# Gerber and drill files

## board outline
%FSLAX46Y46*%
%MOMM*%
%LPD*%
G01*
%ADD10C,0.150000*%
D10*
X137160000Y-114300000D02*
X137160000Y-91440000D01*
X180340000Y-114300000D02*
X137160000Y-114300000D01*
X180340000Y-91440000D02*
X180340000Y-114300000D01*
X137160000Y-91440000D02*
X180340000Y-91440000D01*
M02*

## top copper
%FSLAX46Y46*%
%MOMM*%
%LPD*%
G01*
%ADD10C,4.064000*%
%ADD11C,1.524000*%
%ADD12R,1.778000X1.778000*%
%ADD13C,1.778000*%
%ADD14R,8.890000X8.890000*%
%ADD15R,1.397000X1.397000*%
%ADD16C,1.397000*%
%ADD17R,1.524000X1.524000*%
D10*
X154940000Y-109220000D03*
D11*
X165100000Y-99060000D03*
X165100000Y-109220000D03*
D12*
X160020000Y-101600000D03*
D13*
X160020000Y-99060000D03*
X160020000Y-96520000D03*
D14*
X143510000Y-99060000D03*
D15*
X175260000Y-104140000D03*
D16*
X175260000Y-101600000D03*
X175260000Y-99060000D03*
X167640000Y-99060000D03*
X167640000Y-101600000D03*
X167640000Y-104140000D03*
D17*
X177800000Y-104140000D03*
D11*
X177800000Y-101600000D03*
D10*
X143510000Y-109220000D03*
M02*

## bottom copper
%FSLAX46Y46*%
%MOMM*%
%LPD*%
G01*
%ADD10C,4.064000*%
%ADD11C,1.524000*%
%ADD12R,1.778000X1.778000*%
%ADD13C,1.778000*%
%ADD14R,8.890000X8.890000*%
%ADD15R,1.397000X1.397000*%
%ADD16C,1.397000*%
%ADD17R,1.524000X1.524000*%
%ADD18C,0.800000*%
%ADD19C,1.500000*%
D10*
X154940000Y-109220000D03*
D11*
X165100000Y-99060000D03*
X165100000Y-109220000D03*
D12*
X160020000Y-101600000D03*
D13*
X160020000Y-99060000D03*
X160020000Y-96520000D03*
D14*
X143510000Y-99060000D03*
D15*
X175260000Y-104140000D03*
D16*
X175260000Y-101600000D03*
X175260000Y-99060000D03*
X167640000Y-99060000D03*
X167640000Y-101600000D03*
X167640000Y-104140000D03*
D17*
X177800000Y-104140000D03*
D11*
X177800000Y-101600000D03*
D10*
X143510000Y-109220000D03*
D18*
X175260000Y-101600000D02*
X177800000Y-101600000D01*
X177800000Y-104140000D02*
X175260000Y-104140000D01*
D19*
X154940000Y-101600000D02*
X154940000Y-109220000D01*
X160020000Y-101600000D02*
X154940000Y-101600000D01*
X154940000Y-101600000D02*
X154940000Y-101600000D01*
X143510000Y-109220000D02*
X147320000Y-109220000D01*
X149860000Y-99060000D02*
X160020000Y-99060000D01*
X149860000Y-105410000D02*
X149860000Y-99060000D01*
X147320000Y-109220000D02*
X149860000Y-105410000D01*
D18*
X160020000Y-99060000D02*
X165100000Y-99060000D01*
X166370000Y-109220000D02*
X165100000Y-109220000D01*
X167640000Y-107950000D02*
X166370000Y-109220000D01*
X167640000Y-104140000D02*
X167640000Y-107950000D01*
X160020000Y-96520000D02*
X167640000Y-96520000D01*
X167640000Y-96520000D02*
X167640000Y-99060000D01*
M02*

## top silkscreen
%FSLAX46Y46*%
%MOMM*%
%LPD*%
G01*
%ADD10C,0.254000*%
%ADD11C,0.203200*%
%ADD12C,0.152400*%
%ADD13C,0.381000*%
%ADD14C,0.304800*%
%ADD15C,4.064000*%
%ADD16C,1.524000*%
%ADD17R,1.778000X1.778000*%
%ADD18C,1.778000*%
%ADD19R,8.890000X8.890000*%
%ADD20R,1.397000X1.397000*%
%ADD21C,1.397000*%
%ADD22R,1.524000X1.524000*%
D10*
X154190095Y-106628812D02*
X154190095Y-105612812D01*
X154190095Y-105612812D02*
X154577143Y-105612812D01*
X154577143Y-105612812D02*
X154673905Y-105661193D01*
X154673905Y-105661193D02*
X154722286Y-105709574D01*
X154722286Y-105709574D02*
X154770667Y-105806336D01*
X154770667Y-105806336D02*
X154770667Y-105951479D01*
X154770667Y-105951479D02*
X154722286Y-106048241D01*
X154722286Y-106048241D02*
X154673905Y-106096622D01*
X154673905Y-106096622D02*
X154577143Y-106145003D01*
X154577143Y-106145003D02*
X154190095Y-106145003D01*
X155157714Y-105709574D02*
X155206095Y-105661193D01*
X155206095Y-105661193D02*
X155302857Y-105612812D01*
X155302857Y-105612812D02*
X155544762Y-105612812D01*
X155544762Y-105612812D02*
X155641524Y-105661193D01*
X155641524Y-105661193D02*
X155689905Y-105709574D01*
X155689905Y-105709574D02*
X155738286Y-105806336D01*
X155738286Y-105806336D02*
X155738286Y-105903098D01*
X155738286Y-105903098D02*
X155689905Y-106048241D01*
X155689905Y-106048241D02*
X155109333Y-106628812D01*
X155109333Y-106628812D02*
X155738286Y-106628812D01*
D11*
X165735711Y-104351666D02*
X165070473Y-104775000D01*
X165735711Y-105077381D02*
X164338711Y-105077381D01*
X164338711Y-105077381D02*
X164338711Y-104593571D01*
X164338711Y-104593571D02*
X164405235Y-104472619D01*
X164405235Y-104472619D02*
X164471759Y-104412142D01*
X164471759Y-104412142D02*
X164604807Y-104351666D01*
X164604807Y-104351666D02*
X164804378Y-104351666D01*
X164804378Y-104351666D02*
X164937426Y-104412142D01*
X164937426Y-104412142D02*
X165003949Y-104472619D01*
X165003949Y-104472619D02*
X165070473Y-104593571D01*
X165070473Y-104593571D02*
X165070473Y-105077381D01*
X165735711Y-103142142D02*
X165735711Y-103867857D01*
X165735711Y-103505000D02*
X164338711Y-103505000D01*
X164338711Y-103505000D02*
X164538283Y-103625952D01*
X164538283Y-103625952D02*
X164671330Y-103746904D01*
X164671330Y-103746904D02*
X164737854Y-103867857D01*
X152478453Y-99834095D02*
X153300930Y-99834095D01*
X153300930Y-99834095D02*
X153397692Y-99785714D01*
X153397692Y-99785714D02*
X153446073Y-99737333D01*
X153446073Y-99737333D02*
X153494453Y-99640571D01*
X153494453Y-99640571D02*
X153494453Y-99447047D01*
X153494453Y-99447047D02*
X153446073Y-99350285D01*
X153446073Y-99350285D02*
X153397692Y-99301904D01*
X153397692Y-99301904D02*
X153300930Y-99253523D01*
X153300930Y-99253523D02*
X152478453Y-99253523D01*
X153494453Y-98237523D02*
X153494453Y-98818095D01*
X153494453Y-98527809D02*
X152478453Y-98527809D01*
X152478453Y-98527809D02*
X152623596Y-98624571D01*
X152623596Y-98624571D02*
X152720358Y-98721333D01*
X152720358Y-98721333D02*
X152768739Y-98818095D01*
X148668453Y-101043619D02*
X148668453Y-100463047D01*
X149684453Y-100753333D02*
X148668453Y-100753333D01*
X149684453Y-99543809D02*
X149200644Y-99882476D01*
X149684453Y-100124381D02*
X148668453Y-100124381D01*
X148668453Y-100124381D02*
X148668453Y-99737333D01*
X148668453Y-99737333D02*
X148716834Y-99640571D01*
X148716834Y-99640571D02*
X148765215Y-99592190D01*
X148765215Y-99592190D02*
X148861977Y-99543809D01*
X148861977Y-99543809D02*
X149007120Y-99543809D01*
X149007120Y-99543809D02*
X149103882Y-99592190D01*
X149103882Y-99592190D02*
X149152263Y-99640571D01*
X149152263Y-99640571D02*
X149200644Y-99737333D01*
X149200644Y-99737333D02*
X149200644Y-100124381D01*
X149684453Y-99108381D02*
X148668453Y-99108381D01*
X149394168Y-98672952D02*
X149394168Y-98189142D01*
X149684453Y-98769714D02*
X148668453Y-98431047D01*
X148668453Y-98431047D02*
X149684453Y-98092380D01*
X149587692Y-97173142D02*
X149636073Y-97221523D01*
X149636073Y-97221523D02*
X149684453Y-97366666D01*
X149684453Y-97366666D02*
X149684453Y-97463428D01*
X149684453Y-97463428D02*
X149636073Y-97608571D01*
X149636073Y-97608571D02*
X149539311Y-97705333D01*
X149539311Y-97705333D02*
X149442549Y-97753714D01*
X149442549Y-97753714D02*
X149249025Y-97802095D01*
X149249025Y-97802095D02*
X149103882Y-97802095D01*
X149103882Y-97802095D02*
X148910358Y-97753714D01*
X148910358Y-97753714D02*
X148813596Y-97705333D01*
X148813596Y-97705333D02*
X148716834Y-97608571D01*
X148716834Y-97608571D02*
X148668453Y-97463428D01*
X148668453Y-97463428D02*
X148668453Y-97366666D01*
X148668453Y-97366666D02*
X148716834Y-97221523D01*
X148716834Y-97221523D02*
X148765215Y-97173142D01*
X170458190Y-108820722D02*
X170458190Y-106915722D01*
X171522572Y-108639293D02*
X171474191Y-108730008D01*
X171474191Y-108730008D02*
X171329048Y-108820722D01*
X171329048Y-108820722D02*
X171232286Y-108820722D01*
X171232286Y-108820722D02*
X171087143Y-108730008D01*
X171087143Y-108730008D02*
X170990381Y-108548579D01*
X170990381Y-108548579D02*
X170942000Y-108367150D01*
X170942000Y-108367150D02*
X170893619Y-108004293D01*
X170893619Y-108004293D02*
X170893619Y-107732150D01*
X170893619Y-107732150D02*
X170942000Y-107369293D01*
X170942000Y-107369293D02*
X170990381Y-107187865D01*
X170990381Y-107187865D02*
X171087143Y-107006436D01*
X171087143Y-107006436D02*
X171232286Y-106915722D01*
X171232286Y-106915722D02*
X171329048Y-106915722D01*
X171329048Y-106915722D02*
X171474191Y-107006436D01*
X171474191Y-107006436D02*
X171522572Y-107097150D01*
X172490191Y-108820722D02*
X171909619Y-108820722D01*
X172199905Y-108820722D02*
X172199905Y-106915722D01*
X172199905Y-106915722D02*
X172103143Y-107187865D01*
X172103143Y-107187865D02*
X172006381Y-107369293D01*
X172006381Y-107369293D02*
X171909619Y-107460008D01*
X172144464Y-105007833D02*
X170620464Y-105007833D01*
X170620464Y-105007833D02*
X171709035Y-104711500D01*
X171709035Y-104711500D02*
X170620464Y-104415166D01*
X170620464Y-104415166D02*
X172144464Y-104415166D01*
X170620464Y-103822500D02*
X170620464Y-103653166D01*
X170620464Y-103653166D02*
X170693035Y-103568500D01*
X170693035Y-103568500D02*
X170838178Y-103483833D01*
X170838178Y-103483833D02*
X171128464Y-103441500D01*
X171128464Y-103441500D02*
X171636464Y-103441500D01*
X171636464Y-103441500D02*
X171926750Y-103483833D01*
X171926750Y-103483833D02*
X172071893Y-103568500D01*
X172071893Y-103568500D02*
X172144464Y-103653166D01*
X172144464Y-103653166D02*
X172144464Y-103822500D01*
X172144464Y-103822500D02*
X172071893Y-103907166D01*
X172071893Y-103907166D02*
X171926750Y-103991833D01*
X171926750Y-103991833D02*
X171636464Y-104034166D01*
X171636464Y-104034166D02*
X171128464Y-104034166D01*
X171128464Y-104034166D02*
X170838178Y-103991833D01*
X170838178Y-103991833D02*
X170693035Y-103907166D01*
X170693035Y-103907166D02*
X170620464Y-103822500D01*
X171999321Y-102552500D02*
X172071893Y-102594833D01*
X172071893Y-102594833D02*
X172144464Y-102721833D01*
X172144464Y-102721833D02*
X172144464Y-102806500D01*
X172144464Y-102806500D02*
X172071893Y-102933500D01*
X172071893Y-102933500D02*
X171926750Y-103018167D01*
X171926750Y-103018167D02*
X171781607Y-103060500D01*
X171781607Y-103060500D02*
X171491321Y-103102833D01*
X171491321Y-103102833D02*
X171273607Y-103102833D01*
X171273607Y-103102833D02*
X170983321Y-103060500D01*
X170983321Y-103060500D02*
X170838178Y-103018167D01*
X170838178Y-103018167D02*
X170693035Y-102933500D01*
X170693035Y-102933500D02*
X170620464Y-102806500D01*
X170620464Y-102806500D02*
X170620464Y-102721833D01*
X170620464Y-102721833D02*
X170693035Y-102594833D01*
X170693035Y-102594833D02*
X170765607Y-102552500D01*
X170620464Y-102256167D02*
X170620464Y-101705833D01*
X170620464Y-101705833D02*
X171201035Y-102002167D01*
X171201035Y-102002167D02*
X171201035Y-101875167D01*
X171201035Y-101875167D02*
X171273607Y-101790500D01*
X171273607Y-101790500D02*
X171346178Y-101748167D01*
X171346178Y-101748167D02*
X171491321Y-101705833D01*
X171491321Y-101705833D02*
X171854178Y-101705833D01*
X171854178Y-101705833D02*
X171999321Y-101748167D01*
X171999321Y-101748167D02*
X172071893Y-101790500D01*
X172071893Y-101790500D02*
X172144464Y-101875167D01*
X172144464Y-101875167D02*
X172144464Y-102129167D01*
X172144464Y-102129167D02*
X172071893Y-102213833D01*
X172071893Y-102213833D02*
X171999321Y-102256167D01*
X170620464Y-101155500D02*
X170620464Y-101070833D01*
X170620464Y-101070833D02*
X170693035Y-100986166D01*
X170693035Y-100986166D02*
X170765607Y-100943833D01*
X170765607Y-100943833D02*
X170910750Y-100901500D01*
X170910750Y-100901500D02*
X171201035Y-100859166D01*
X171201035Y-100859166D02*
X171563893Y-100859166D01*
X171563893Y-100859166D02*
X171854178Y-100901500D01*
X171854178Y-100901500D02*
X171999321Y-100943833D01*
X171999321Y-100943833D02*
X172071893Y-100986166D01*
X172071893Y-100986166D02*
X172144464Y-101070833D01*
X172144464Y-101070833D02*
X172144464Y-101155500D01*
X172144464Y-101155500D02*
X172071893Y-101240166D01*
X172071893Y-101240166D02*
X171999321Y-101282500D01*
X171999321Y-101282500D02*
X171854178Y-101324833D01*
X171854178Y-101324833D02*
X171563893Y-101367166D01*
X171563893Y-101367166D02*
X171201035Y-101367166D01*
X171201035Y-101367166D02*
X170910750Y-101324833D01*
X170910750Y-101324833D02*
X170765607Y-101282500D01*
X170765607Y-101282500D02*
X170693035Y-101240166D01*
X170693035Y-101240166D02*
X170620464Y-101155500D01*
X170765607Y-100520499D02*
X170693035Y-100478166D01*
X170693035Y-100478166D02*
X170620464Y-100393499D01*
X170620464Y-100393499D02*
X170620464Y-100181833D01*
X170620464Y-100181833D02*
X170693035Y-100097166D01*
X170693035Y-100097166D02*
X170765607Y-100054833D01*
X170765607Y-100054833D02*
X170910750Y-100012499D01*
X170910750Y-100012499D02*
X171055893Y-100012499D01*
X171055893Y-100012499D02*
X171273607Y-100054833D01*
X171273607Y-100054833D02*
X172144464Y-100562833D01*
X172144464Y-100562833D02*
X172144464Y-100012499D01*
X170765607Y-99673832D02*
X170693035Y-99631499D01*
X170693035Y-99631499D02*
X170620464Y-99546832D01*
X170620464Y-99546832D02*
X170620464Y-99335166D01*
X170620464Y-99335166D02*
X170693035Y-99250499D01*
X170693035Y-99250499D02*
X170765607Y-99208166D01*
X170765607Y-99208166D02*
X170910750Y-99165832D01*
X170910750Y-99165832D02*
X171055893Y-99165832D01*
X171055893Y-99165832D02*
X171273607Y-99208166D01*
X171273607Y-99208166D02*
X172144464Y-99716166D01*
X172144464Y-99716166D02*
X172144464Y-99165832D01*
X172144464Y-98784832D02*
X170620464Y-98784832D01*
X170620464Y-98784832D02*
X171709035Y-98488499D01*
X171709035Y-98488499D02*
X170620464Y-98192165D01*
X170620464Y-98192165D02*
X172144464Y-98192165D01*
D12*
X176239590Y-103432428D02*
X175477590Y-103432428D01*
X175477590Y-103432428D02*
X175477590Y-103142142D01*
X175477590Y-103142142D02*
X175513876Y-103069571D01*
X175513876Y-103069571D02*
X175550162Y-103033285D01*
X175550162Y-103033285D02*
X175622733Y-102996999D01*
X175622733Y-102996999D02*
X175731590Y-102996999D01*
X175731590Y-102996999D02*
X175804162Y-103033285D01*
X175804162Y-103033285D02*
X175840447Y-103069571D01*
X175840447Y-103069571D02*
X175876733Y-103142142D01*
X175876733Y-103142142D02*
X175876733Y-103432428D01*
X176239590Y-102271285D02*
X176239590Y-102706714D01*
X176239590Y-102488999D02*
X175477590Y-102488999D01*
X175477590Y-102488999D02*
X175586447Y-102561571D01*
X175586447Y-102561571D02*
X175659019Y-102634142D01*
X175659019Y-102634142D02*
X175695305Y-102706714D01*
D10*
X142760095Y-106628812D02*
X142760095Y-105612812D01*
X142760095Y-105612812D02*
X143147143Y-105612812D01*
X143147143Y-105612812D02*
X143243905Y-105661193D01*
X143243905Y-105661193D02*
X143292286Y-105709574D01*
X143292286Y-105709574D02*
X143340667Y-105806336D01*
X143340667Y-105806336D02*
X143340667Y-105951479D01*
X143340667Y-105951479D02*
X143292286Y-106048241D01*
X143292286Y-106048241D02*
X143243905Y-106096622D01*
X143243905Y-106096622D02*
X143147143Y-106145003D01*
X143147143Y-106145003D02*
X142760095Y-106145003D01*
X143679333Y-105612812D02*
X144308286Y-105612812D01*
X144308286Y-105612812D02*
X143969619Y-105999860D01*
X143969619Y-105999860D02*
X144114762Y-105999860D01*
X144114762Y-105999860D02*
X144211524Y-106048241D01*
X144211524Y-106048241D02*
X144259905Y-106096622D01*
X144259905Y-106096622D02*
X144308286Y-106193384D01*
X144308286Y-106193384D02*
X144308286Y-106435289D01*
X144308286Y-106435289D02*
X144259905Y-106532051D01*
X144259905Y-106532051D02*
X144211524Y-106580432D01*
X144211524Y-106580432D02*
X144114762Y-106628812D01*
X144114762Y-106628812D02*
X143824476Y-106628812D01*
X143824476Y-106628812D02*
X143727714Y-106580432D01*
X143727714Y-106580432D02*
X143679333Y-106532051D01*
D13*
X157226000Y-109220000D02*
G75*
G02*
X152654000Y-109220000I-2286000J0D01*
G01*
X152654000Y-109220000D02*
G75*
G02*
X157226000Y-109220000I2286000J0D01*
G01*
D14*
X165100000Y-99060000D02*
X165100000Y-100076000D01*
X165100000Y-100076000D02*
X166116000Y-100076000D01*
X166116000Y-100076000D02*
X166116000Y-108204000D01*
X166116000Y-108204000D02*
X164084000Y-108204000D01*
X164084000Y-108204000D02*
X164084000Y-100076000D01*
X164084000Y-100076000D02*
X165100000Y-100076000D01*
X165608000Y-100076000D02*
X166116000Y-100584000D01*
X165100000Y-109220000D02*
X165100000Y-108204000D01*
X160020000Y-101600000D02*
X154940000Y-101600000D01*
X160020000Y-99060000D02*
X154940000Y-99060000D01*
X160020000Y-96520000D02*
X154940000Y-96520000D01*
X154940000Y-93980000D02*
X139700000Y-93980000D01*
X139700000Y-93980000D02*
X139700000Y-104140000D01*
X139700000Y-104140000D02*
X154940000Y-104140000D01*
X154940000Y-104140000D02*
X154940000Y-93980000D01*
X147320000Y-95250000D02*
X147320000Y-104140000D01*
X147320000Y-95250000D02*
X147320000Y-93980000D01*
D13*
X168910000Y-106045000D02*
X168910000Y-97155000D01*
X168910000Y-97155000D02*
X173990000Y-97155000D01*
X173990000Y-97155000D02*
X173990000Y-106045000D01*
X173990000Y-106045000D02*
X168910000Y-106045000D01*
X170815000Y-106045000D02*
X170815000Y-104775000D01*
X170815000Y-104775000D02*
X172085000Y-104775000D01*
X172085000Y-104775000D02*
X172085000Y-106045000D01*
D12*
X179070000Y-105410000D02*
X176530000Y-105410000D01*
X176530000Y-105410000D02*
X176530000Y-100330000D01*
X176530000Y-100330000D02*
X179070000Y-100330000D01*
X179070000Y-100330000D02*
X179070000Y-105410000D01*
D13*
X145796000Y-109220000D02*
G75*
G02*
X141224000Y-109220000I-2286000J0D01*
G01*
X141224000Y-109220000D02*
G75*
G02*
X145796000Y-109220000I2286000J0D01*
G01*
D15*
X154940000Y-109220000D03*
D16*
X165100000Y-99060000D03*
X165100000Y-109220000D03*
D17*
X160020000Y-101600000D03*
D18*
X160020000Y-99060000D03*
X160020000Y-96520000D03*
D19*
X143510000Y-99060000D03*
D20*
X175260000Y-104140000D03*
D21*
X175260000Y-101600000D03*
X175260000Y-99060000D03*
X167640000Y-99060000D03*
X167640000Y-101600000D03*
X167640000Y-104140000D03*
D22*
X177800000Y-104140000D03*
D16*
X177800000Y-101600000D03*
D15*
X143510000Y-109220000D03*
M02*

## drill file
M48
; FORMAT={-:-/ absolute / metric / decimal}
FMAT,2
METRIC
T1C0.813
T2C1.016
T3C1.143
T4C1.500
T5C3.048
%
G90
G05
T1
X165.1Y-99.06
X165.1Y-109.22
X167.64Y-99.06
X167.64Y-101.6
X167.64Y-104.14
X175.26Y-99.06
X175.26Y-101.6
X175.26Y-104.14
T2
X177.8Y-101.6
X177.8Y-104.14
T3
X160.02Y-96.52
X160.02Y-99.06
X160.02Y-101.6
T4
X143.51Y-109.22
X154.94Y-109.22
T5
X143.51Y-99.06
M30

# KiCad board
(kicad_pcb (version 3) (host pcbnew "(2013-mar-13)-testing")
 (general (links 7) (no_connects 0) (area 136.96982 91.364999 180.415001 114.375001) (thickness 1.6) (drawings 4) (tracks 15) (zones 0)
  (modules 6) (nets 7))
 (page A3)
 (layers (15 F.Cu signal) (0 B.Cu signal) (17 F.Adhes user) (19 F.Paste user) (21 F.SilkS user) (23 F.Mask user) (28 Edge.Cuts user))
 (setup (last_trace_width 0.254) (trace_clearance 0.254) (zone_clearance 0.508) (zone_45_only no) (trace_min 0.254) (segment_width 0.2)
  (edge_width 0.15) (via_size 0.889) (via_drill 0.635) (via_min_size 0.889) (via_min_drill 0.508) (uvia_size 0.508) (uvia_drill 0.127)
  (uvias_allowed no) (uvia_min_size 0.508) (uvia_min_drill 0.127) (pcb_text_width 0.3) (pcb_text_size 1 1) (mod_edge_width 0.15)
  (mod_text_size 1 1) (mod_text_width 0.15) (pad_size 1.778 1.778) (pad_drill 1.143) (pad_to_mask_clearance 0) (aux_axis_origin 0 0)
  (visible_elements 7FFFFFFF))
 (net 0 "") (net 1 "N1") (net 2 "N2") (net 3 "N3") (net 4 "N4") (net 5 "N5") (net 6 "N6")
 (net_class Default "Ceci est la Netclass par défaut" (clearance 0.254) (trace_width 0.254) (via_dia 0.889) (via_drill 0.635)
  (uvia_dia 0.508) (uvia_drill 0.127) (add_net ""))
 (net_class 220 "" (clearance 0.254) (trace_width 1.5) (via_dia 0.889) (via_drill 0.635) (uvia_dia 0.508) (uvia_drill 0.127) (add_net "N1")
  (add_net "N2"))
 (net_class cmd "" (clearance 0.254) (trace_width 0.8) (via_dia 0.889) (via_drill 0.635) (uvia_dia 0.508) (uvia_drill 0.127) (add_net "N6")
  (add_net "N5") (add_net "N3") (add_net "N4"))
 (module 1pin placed (layer F.Cu) (at 154.94 109.22)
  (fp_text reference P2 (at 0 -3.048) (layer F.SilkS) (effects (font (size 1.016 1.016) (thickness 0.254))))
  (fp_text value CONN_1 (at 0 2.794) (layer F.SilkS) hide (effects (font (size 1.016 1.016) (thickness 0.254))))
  (fp_circle (center 0 0) (end 0 -2.286) (layer F.SilkS) (width 0.381))
  (pad 1 thru_hole circle (at 0 0) (size 4.064 4.064) (drill 1.5) (layers *.Cu *.Mask F.SilkS) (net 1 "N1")))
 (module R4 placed (layer F.Cu) (at 165.1 104.14 270) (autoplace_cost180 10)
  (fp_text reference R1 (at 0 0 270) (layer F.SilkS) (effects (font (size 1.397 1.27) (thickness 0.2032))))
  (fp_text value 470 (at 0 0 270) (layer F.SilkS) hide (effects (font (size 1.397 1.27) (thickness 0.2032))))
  (fp_line (start -5.08 0) (end -4.064 0) (layer F.SilkS) (width 0.3048))
  (fp_line (start -4.064 0) (end -4.064 -1.016) (layer F.SilkS) (width 0.3048))
  (fp_line (start -4.064 -1.016) (end 4.064 -1.016) (layer F.SilkS) (width 0.3048))
  (fp_line (start 4.064 -1.016) (end 4.064 1.016) (layer F.SilkS) (width 0.3048))
  (fp_line (start 4.064 1.016) (end -4.064 1.016) (layer F.SilkS) (width 0.3048))
  (fp_line (start -4.064 1.016) (end -4.064 0) (layer F.SilkS) (width 0.3048))
  (fp_line (start -4.064 -0.508) (end -3.556 -1.016) (layer F.SilkS) (width 0.3048))
  (fp_line (start 5.08 0) (end 4.064 0) (layer F.SilkS) (width 0.3048))
  (pad 1 thru_hole circle (at -5.08 0 270) (size 1.524 1.524) (drill 0.8128) (layers *.Cu *.Mask F.SilkS) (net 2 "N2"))
  (pad 2 thru_hole circle (at 5.08 0 270) (size 1.524 1.524) (drill 0.8128) (layers *.Cu *.Mask F.SilkS) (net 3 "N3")))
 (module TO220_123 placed (layer F.Cu) (at 160.02 99.06 180)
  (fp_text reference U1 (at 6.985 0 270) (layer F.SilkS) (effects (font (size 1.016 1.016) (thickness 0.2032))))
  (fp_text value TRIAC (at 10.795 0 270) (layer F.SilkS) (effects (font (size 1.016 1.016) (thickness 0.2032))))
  (fp_line (start 0 -2.54) (end 5.08 -2.54) (layer F.SilkS) (width 0.3048))
  (fp_line (start 0 0) (end 5.08 0) (layer F.SilkS) (width 0.3048))
  (fp_line (start 0 2.54) (end 5.08 2.54) (layer F.SilkS) (width 0.3048))
  (fp_line (start 5.08 5.08) (end 20.32 5.08) (layer F.SilkS) (width 0.3048))
  (fp_line (start 20.32 5.08) (end 20.32 -5.08) (layer F.SilkS) (width 0.3048))
  (fp_line (start 20.32 -5.08) (end 5.08 -5.08) (layer F.SilkS) (width 0.3048))
  (fp_line (start 5.08 -5.08) (end 5.08 5.08) (layer F.SilkS) (width 0.3048))
  (fp_line (start 12.7 3.81) (end 12.7 -5.08) (layer F.SilkS) (width 0.3048))
  (fp_line (start 12.7 3.81) (end 12.7 5.08) (layer F.SilkS) (width 0.3048))
  (pad 1 thru_hole rect (at 0 -2.54 180) (size 1.778 1.778) (drill 1.143) (layers *.Cu *.Mask F.SilkS) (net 1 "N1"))
  (pad 2 thru_hole circle (at 0 0 180) (size 1.778 1.778) (drill 1.143) (layers *.Cu *.Mask F.SilkS) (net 2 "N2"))
  (pad 3 thru_hole circle (at 0 2.54 180) (size 1.778 1.778) (drill 1.143) (layers *.Cu *.Mask F.SilkS) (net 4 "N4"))
  (pad 4 thru_hole rect (at 16.51 0 180) (size 8.89 8.89) (drill 3.048) (layers *.Cu *.SilkS *.Mask)))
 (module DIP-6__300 (layer F.Cu) (at 171.45 101.6 90)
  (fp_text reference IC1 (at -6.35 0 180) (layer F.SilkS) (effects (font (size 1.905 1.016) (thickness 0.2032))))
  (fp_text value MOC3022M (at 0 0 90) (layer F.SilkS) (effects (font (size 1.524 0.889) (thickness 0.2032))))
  (fp_line (start -4.445 -2.54) (end 4.445 -2.54) (layer F.SilkS) (width 0.381))
  (fp_line (start 4.445 -2.54) (end 4.445 2.54) (layer F.SilkS) (width 0.381))
  (fp_line (start 4.445 2.54) (end -4.445 2.54) (layer F.SilkS) (width 0.381))
  (fp_line (start -4.445 2.54) (end -4.445 -2.54) (layer F.SilkS) (width 0.381))
  (fp_line (start -4.445 -0.635) (end -3.175 -0.635) (layer F.SilkS) (width 0.381))
  (fp_line (start -3.175 -0.635) (end -3.175 0.635) (layer F.SilkS) (width 0.381))
  (fp_line (start -3.175 0.635) (end -4.445 0.635) (layer F.SilkS) (width 0.381))
  (pad 1 thru_hole rect (at -2.54 3.81 90) (size 1.397 1.397) (drill 0.8128) (layers *.Cu *.Mask F.SilkS) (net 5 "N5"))
  (pad 2 thru_hole circle (at 0 3.81 90) (size 1.397 1.397) (drill 0.8128) (layers *.Cu *.Mask F.SilkS) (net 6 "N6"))
  (pad 3 thru_hole circle (at 2.54 3.81 90) (size 1.397 1.397) (drill 0.8128) (layers *.Cu *.Mask F.SilkS))
  (pad 4 thru_hole circle (at 2.54 -3.81 90) (size 1.397 1.397) (drill 0.8128) (layers *.Cu *.Mask F.SilkS) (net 4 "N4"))
  (pad 5 thru_hole circle (at 0 -3.81 90) (size 1.397 1.397) (drill 0.8128) (layers *.Cu *.Mask F.SilkS))
  (pad 6 thru_hole circle (at -2.54 -3.81 90) (size 1.397 1.397) (drill 0.8128) (layers *.Cu *.Mask F.SilkS) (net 3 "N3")))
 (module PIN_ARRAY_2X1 (layer F.Cu) (at 177.8 102.87 90)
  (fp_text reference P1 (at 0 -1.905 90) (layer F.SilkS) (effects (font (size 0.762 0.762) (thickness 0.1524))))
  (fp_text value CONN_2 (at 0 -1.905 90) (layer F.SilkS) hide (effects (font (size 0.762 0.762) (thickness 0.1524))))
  (fp_line (start -2.54 1.27) (end -2.54 -1.27) (layer F.SilkS) (width 0.1524))
  (fp_line (start -2.54 -1.27) (end 2.54 -1.27) (layer F.SilkS) (width 0.1524))
  (fp_line (start 2.54 -1.27) (end 2.54 1.27) (layer F.SilkS) (width 0.1524))
  (fp_line (start 2.54 1.27) (end -2.54 1.27) (layer F.SilkS) (width 0.1524))
  (pad 1 thru_hole rect (at -1.27 0 90) (size 1.524 1.524) (drill 1.016) (layers *.Cu *.Mask F.SilkS) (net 5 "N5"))
  (pad 2 thru_hole circle (at 1.27 0 90) (size 1.524 1.524) (drill 1.016) (layers *.Cu *.Mask F.SilkS) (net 6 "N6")))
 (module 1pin (layer F.Cu) (at 143.51 109.22)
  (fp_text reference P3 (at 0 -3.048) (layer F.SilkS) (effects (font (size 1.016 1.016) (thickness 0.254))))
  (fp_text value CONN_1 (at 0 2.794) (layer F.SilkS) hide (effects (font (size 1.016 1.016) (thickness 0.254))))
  (fp_circle (center 0 0) (end 0 -2.286) (layer F.SilkS) (width 0.381))
  (pad 1 thru_hole circle (at 0 0) (size 4.064 4.064) (drill 1.5) (layers *.Cu *.Mask F.SilkS) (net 2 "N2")))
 (gr_line (start 137.16 114.3) (end 137.16 91.44) (angle 90) (layer Edge.Cuts) (width 0.15))
 (gr_line (start 180.34 114.3) (end 137.16 114.3) (angle 90) (layer Edge.Cuts) (width 0.15))
 (gr_line (start 180.34 91.44) (end 180.34 114.3) (angle 90) (layer Edge.Cuts) (width 0.15))
 (gr_line (start 137.16 91.44) (end 180.34 91.44) (angle 90) (layer Edge.Cuts) (width 0.15))
 (segment (start 175.26 101.6) (end 177.8 101.6) (width 0.8) (layer B.Cu) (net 6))
 (segment (start 177.8 104.14) (end 175.26 104.14) (width 0.8) (layer B.Cu) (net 5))
 (segment (start 154.94 101.6) (end 154.94 109.22) (width 1.5) (layer B.Cu) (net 1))
 (segment (start 160.02 101.6) (end 154.94 101.6) (width 1.5) (layer B.Cu) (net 1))
 (segment (start 154.94 101.6) (end 154.94 101.6) (width 1.5) (layer B.Cu) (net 1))
 (segment (start 143.51 109.22) (end 147.32 109.22) (width 1.5) (layer B.Cu) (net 2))
 (segment (start 149.86 99.06) (end 160.02 99.06) (width 1.5) (layer B.Cu) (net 2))
 (segment (start 149.86 105.41) (end 149.86 99.06) (width 1.5) (layer B.Cu) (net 2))
 (segment (start 147.32 109.22) (end 149.86 105.41) (width 1.5) (layer B.Cu) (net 2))
 (segment (start 160.02 99.06) (end 165.1 99.06) (width 0.8) (layer B.Cu) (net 2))
 (segment (start 166.37 109.22) (end 165.1 109.22) (width 0.8) (layer B.Cu) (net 3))
 (segment (start 167.64 107.95) (end 166.37 109.22) (width 0.8) (layer B.Cu) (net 3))
 (segment (start 167.64 104.14) (end 167.64 107.95) (width 0.8) (layer B.Cu) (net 3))
 (segment (start 160.02 96.52) (end 167.64 96.52) (width 0.8) (layer B.Cu) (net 4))
 (segment (start 167.64 96.52) (end 167.64 99.06) (width 0.8) (layer B.Cu) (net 4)))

